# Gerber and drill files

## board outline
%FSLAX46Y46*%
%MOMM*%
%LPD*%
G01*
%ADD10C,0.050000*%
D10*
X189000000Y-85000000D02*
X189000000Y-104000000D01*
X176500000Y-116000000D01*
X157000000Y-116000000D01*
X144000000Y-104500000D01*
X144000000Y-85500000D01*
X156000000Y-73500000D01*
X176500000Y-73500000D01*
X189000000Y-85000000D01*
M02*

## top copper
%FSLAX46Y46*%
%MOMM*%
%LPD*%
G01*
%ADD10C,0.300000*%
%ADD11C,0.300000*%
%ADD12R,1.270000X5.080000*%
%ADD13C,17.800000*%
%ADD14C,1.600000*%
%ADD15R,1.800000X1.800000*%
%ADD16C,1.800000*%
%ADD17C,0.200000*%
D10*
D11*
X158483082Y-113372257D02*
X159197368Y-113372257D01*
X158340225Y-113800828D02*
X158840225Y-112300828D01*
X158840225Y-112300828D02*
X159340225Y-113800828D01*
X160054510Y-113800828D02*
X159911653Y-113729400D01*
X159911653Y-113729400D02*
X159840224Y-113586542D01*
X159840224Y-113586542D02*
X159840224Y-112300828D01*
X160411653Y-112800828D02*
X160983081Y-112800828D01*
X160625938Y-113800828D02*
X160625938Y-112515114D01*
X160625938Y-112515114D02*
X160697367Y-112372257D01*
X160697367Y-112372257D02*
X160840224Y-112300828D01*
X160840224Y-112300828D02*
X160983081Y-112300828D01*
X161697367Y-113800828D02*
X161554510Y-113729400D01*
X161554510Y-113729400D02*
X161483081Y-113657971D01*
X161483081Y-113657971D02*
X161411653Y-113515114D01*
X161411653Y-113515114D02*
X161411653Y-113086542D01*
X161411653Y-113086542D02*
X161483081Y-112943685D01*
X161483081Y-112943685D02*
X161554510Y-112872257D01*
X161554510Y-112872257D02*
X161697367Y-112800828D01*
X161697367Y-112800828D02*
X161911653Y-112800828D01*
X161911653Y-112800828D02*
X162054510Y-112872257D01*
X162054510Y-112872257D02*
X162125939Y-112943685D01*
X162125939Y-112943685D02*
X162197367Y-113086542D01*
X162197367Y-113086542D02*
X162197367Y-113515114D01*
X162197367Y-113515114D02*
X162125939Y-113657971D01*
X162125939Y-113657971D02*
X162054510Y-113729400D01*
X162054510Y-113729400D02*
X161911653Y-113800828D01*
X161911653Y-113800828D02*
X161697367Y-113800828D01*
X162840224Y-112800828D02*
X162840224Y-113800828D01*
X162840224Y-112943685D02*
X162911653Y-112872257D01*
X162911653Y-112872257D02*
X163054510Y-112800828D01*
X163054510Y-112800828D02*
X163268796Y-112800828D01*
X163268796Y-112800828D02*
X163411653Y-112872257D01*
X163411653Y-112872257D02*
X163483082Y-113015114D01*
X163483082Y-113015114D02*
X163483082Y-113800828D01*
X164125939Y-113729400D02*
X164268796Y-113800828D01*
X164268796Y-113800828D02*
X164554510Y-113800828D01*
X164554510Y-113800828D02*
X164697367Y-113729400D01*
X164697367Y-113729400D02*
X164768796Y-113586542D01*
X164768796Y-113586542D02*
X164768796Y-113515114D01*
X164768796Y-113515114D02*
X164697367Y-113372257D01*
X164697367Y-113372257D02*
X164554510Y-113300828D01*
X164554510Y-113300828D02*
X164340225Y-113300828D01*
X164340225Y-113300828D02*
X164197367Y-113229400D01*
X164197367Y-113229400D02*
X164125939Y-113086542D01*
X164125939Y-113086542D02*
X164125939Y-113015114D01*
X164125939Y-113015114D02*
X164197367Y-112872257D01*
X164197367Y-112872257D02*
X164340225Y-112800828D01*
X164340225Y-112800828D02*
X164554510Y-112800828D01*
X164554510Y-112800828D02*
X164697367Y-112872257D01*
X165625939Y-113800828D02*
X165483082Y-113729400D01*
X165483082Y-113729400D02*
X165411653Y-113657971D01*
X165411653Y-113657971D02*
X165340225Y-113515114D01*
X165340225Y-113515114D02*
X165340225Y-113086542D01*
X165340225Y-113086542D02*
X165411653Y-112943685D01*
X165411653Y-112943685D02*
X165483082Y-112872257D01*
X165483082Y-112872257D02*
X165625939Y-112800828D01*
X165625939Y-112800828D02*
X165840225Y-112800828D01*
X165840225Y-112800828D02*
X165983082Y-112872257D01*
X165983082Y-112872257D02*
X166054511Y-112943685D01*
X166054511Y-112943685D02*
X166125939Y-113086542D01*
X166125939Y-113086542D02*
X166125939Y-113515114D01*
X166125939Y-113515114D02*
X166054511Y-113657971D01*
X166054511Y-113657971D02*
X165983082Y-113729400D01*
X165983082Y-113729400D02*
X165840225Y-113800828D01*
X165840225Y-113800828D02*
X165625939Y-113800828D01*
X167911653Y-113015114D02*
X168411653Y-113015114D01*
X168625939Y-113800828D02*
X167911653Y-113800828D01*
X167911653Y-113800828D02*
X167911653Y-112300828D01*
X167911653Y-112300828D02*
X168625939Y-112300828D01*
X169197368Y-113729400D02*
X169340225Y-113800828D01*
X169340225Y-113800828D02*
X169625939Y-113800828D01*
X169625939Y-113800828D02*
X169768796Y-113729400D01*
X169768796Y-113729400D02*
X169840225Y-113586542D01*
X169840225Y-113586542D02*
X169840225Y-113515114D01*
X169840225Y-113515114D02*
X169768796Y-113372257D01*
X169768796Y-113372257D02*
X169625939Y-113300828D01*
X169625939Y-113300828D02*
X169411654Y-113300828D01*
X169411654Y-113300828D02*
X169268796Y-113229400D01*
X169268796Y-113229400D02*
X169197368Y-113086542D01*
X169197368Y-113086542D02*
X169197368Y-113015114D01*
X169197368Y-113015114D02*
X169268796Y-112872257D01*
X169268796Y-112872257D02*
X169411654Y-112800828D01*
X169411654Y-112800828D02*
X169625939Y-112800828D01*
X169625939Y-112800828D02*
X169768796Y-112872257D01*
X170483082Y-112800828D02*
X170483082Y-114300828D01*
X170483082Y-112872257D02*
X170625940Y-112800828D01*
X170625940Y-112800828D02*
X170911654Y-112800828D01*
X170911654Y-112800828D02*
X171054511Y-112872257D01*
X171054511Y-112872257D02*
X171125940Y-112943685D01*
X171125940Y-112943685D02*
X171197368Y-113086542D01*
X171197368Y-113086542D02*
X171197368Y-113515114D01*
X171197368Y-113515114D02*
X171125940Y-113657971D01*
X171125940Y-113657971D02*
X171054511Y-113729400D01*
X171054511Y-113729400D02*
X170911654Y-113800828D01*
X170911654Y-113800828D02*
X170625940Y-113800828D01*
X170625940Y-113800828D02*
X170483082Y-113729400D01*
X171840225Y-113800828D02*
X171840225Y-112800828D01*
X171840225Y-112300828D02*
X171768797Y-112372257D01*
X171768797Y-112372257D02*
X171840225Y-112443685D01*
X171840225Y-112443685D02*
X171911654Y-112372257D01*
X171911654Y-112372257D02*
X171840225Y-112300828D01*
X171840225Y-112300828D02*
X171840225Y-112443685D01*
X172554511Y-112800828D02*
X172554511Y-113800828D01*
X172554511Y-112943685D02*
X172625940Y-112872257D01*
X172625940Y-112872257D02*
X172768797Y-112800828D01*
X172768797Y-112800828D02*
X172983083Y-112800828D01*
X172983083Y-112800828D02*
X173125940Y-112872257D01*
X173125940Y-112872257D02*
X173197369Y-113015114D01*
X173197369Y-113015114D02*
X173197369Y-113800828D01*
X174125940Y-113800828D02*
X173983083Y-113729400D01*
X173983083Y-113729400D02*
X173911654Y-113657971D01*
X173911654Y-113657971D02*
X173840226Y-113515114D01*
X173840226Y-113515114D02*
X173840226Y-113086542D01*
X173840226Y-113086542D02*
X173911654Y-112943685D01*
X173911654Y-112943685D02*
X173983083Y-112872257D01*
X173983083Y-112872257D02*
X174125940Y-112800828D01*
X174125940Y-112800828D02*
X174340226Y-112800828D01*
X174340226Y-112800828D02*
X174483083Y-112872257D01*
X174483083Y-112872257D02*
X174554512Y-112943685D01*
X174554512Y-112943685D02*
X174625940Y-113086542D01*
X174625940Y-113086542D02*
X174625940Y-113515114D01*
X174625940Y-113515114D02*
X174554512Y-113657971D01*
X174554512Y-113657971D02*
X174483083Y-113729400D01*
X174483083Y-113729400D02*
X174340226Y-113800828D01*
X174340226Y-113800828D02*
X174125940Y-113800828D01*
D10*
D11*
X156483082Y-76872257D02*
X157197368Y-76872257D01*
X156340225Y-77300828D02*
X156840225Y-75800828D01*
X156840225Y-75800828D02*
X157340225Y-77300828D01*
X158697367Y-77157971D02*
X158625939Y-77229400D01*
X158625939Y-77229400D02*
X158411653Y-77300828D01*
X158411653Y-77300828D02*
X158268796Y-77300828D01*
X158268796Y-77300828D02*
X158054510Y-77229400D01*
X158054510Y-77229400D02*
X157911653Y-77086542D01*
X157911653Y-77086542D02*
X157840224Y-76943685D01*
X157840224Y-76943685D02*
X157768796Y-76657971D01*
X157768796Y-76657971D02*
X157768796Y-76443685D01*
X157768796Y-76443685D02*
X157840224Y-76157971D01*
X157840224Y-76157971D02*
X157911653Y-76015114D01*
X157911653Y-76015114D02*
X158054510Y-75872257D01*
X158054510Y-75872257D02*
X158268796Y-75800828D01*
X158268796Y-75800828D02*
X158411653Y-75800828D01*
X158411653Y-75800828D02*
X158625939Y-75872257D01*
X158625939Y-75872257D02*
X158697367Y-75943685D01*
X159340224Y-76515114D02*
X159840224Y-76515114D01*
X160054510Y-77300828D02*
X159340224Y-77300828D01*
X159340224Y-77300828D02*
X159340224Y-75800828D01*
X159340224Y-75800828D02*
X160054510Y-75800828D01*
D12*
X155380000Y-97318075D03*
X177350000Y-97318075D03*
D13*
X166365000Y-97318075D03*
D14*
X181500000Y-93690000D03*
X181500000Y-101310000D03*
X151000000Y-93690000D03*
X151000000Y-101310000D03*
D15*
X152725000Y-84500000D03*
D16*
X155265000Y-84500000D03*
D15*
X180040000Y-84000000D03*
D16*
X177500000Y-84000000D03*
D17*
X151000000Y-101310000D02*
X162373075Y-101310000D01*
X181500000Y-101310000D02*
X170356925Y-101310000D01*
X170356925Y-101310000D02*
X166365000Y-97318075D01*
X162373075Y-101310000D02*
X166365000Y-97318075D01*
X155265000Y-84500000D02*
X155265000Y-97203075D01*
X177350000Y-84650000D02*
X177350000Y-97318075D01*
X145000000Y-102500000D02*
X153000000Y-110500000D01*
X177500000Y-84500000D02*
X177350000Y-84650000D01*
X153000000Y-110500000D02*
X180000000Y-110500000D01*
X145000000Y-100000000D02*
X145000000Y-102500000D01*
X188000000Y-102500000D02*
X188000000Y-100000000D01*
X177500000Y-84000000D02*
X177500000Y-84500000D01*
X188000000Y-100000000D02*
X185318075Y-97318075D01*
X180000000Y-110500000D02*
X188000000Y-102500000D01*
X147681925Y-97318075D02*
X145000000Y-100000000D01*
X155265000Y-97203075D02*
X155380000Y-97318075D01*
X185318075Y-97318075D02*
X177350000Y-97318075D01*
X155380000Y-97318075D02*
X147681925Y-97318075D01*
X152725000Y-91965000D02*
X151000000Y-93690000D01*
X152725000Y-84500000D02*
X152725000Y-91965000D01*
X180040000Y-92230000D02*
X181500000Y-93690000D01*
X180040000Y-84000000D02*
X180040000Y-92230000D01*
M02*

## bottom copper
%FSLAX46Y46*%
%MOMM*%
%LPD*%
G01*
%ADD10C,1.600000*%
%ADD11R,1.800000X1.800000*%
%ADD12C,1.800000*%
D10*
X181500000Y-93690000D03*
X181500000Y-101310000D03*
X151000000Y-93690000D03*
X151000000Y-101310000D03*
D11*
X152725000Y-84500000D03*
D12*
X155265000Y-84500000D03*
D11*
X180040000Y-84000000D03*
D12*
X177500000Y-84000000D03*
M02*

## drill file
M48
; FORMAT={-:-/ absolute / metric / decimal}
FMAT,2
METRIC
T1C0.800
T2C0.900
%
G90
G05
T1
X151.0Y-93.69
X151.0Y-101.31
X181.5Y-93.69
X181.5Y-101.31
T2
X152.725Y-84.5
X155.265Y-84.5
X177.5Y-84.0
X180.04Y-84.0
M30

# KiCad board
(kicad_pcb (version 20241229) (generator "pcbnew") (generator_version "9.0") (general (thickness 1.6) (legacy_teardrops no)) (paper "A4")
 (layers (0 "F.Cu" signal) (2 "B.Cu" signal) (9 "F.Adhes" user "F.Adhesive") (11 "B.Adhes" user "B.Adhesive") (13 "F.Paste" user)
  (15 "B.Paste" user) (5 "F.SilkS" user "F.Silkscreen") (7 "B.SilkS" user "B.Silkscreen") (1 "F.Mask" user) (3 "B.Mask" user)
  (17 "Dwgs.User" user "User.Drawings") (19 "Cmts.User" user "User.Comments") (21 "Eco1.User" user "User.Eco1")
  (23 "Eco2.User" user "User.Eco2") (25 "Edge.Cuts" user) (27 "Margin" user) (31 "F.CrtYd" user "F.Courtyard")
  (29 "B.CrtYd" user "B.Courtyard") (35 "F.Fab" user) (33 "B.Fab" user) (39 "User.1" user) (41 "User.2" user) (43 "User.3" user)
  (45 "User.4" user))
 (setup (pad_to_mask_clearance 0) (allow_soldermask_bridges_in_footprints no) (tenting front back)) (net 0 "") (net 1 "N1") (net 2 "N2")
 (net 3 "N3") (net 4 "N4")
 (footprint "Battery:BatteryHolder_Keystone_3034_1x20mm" (layer "F.Cu") (at 166.365 97.318075)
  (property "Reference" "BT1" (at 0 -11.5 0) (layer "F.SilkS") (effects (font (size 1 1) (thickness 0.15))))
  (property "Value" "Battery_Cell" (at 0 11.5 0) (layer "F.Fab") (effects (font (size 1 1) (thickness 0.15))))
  (pad "1" smd rect (at -10.985 0) (size 1.27 5.08) (layers "F.Cu" "F.Mask" "F.Paste") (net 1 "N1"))
  (pad "1" smd rect (at 10.985 0) (size 1.27 5.08) (layers "F.Cu" "F.Mask" "F.Paste") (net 1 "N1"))
  (pad "2" smd circle (at 0 0) (size 17.8 17.8) (layers "F.Cu" "F.Mask") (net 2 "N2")))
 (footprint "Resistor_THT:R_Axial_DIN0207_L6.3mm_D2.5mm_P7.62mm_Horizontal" (layer "F.Cu") (at 181.5 93.69 -90)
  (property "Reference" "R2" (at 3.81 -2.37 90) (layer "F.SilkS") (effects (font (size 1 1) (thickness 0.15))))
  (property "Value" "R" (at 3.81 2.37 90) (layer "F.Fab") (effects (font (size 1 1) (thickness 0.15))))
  (pad "1" thru_hole circle (at 0 0 270) (size 1.6 1.6) (drill 0.8) (layers "*.Cu" "*.Mask") (remove_unused_layers no) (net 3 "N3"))
  (pad "2" thru_hole circle (at 7.62 0 270) (size 1.6 1.6) (drill 0.8) (layers "*.Cu" "*.Mask") (remove_unused_layers no) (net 2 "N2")))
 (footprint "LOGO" (layer "F.Cu") (at 170 80)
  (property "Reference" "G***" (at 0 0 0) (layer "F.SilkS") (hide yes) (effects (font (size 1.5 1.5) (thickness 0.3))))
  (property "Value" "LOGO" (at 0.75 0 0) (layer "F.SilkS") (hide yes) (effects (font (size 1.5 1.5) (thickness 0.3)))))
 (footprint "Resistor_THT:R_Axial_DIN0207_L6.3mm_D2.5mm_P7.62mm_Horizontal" (layer "F.Cu") (at 151 93.69 -90)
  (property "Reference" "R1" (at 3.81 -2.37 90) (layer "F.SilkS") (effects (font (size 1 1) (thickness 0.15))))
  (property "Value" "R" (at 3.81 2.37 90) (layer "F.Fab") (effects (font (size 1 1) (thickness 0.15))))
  (pad "1" thru_hole circle (at 0 0 270) (size 1.6 1.6) (drill 0.8) (layers "*.Cu" "*.Mask") (remove_unused_layers no) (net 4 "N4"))
  (pad "2" thru_hole circle (at 7.62 0 270) (size 1.6 1.6) (drill 0.8) (layers "*.Cu" "*.Mask") (remove_unused_layers no) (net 2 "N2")))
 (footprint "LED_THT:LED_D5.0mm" (layer "F.Cu") (at 152.725 84.5)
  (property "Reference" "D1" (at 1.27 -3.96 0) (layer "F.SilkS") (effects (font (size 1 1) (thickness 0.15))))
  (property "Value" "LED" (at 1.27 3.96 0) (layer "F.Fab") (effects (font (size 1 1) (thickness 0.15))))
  (pad "1" thru_hole rect (at 0 0) (size 1.8 1.8) (drill 0.9) (layers "*.Cu" "*.Mask") (remove_unused_layers no) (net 4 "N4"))
  (pad "2" thru_hole circle (at 2.54 0) (size 1.8 1.8) (drill 0.9) (layers "*.Cu" "*.Mask") (remove_unused_layers no) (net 1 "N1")))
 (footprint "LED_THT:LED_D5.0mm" (layer "F.Cu") (at 180.04 84 180)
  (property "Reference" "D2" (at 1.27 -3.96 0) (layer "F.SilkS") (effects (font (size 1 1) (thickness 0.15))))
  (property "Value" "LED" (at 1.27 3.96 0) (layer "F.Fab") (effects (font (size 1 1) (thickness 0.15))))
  (pad "1" thru_hole rect (at 0 0 180) (size 1.8 1.8) (drill 0.9) (layers "*.Cu" "*.Mask") (remove_unused_layers no) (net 3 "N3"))
  (pad "2" thru_hole circle (at 2.54 0 180) (size 1.8 1.8) (drill 0.9) (layers "*.Cu" "*.Mask") (remove_unused_layers no) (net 1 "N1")))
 (gr_poly
  (pts (xy 189 85) (xy 189 104) (xy 176.5 116) (xy 157 116) (xy 144 104.5) (xy 144 85.5) (xy 156 73.5) (xy 176.5 73.5))
  (stroke (width 0.05) (type solid)) (fill no) (layer "Edge.Cuts"))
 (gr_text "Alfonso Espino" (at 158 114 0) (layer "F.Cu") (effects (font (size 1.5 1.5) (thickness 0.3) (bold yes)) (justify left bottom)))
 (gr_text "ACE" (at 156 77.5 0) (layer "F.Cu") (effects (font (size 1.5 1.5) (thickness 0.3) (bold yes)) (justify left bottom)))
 (segment (start 151 101.31) (end 162.373075 101.31) (width 0.2) (layer "F.Cu") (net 2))
 (segment (start 181.5 101.31) (end 170.356925 101.31) (width 0.2) (layer "F.Cu") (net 2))
 (segment (start 170.356925 101.31) (end 166.365 97.318075) (width 0.2) (layer "F.Cu") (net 2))
 (segment (start 162.373075 101.31) (end 166.365 97.318075) (width 0.2) (layer "F.Cu") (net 2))
 (segment (start 155.265 84.5) (end 155.265 97.203075) (width 0.2) (layer "F.Cu") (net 1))
 (segment (start 177.35 84.65) (end 177.35 97.318075) (width 0.2) (layer "F.Cu") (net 1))
 (segment (start 145 102.5) (end 153 110.5) (width 0.2) (layer "F.Cu") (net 1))
 (segment (start 177.5 84.5) (end 177.35 84.65) (width 0.2) (layer "F.Cu") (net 1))
 (segment (start 153 110.5) (end 180 110.5) (width 0.2) (layer "F.Cu") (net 1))
 (segment (start 145 100) (end 145 102.5) (width 0.2) (layer "F.Cu") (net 1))
 (segment (start 188 102.5) (end 188 100) (width 0.2) (layer "F.Cu") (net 1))
 (segment (start 177.5 84) (end 177.5 84.5) (width 0.2) (layer "F.Cu") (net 1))
 (segment (start 188 100) (end 185.318075 97.318075) (width 0.2) (layer "F.Cu") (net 1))
 (segment (start 180 110.5) (end 188 102.5) (width 0.2) (layer "F.Cu") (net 1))
 (segment (start 147.681925 97.318075) (end 145 100) (width 0.2) (layer "F.Cu") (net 1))
 (segment (start 155.265 97.203075) (end 155.38 97.318075) (width 0.2) (layer "F.Cu") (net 1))
 (segment (start 185.318075 97.318075) (end 177.35 97.318075) (width 0.2) (layer "F.Cu") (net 1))
 (segment (start 155.38 97.318075) (end 147.681925 97.318075) (width 0.2) (layer "F.Cu") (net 1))
 (segment (start 152.725 91.965) (end 151 93.69) (width 0.2) (layer "F.Cu") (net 4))
 (segment (start 152.725 84.5) (end 152.725 91.965) (width 0.2) (layer "F.Cu") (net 4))
 (segment (start 180.04 92.23) (end 181.5 93.69) (width 0.2) (layer "F.Cu") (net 3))
 (segment (start 180.04 84) (end 180.04 92.23) (width 0.2) (layer "F.Cu") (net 3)))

